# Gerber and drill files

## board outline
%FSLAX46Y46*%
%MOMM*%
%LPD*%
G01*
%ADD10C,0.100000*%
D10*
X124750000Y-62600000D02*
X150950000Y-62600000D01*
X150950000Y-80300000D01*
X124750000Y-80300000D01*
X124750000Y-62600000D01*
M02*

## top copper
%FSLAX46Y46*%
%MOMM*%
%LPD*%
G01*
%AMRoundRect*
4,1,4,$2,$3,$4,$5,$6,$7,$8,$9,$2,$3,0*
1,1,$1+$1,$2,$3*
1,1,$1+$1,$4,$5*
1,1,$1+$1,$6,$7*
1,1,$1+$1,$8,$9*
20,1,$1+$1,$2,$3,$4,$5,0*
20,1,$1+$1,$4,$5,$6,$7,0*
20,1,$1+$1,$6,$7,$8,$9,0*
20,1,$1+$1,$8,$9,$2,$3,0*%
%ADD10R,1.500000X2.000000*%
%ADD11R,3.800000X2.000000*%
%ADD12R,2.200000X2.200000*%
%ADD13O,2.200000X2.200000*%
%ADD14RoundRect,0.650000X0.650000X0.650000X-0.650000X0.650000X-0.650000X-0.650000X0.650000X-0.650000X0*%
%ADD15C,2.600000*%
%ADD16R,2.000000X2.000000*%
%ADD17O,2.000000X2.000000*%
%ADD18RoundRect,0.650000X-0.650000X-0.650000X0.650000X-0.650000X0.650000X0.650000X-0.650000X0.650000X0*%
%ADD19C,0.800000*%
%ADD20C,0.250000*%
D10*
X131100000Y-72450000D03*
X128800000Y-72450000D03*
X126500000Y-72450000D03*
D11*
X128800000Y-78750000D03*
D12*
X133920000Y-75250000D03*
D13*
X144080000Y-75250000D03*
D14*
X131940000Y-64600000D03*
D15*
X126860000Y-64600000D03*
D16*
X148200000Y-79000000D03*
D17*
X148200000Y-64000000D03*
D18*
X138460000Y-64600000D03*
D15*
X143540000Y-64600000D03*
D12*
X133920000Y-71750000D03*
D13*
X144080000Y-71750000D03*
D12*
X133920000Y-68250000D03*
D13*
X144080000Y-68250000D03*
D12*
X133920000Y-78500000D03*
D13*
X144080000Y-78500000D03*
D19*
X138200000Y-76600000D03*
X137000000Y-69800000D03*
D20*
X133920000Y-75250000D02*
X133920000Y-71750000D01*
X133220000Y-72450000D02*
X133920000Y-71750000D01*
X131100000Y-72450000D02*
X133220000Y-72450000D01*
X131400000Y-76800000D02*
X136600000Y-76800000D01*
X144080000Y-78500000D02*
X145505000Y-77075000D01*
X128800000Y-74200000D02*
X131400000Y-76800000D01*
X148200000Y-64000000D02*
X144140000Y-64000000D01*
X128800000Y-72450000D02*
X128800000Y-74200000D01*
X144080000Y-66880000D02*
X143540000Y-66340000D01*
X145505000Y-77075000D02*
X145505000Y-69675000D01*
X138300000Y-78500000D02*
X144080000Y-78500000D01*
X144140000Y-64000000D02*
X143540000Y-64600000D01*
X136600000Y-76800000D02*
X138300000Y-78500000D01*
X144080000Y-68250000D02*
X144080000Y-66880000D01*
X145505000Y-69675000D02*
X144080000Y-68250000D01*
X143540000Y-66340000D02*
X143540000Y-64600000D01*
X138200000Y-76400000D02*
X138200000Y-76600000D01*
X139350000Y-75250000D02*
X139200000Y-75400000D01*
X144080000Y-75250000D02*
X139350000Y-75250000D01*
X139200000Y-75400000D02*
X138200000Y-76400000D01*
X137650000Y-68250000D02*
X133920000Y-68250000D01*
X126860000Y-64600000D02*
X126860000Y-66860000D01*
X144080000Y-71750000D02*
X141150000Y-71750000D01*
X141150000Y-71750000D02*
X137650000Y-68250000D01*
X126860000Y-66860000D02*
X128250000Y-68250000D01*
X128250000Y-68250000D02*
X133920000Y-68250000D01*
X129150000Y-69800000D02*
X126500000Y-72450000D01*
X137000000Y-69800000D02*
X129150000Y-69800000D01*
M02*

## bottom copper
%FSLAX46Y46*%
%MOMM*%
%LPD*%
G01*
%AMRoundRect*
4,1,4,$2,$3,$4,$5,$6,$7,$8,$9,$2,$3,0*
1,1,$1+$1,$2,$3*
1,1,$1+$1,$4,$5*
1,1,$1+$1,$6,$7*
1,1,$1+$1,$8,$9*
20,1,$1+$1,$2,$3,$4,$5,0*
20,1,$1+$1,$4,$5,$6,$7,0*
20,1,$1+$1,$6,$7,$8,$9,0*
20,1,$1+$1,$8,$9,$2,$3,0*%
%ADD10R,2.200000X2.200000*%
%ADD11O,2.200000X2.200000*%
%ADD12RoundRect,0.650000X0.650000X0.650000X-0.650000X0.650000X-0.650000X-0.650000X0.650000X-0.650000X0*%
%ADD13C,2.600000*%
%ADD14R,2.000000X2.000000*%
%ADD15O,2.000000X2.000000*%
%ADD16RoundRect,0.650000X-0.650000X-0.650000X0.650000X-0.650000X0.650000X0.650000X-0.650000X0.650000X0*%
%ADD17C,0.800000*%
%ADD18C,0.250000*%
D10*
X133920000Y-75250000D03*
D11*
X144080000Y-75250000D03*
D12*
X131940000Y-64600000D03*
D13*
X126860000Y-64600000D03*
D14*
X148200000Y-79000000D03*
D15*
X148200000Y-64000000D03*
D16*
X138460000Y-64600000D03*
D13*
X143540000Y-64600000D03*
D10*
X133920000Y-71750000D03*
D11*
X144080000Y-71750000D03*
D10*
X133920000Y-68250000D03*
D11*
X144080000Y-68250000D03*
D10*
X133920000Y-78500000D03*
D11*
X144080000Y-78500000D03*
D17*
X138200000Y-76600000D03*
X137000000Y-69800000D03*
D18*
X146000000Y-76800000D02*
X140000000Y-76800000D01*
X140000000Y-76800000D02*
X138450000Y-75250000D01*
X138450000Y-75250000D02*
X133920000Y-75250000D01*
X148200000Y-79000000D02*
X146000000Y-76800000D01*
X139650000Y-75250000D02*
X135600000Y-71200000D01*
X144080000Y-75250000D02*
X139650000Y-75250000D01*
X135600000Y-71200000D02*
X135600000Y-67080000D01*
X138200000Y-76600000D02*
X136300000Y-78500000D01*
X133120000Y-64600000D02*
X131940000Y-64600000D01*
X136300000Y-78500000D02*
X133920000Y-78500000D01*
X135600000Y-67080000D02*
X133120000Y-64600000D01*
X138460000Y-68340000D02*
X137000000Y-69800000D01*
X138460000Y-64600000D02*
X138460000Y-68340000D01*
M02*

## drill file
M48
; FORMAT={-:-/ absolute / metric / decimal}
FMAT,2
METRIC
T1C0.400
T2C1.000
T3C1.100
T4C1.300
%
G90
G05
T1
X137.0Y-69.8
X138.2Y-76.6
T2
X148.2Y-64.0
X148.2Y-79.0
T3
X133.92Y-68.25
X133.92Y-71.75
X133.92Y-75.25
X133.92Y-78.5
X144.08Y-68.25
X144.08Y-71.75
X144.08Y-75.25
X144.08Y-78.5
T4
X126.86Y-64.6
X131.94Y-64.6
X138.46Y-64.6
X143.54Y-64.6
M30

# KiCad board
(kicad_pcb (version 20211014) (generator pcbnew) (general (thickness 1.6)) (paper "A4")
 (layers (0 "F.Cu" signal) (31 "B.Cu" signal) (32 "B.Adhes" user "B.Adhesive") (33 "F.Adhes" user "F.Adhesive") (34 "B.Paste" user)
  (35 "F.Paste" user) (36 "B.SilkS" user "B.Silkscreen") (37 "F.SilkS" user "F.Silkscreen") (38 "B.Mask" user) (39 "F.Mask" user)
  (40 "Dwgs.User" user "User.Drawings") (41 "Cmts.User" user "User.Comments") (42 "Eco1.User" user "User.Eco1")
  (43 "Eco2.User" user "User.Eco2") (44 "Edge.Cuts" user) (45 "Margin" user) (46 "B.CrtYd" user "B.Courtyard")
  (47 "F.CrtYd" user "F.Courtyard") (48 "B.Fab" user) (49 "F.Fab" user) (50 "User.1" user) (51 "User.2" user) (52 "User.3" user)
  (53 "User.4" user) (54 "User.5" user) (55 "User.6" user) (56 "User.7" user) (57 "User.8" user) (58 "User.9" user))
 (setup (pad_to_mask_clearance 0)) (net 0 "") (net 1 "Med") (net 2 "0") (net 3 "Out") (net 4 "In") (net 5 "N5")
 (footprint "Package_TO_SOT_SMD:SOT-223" (layer "F.Cu") (at 128.8 75.6 -90)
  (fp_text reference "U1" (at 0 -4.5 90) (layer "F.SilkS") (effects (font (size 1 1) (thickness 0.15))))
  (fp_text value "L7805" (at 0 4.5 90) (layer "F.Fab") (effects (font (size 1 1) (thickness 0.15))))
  (pad "1" smd rect (at -3.15 -2.3 270) (size 2 1.5) (layers "F.Cu" "F.Paste" "F.Mask") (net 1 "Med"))
  (pad "2" smd rect (at -3.15 0 270) (size 2 1.5) (layers "F.Cu" "F.Paste" "F.Mask") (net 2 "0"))
  (pad "3" smd rect (at -3.15 2.3 270) (size 2 1.5) (layers "F.Cu" "F.Paste" "F.Mask") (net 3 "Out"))
  (pad "4" smd rect (at 3.15 0 270) (size 2 3.8) (layers "F.Cu" "F.Paste" "F.Mask")))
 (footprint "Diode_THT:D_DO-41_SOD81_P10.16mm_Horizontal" (layer "F.Cu") (at 133.92 75.25)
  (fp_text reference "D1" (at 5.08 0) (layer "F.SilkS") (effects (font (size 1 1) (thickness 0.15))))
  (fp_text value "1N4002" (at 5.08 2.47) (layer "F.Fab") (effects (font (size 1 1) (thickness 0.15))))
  (pad "1" thru_hole rect (at 0 0) (size 2.2 2.2) (drill 1.1) (layers *.Cu *.Mask) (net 1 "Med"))
  (pad "2" thru_hole oval (at 10.16 0) (size 2.2 2.2) (drill 1.1) (layers *.Cu *.Mask) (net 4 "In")))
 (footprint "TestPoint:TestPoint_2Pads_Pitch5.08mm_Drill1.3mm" (layer "F.Cu") (at 131.94 64.6 180)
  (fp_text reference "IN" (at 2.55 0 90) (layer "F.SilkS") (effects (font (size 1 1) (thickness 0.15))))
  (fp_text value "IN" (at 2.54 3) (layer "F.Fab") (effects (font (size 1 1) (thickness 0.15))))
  (pad "1" thru_hole roundrect (at 0 0 180) (size 2.6 2.6) (drill 1.3) (layers *.Cu *.Mask) (roundrect_rratio 0.25) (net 4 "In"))
  (pad "2" thru_hole circle (at 5.08 0 180) (size 2.6 2.6) (drill 1.3) (layers *.Cu *.Mask) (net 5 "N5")))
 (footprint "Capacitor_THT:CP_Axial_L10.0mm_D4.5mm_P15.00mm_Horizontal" (layer "F.Cu") (at 148.2 79 90)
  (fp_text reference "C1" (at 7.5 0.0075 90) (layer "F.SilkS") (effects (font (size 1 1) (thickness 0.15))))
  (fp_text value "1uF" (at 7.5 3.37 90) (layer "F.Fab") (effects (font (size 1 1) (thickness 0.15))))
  (pad "1" thru_hole rect (at 0 0 90) (size 2 2) (drill 1) (layers *.Cu *.Mask) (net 1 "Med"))
  (pad "2" thru_hole oval (at 15 0 90) (size 2 2) (drill 1) (layers *.Cu *.Mask) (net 2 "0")))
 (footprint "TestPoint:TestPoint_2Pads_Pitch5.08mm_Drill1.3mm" (layer "F.Cu") (at 138.46 64.6)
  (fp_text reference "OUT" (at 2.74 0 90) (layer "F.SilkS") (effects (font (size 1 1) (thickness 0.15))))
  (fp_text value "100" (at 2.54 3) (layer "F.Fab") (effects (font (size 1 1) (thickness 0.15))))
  (pad "1" thru_hole roundrect (at 0 0) (size 2.6 2.6) (drill 1.3) (layers *.Cu *.Mask) (roundrect_rratio 0.25) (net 3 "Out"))
  (pad "2" thru_hole circle (at 5.08 0) (size 2.6 2.6) (drill 1.3) (layers *.Cu *.Mask) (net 2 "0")))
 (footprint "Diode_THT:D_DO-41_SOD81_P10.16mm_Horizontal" (layer "F.Cu") (at 133.92 71.75)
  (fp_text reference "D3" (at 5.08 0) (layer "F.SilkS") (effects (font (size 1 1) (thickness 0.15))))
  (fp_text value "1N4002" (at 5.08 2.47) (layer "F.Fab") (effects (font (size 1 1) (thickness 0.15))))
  (pad "1" thru_hole rect (at 0 0) (size 2.2 2.2) (drill 1.1) (layers *.Cu *.Mask) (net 1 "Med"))
  (pad "2" thru_hole oval (at 10.16 0) (size 2.2 2.2) (drill 1.1) (layers *.Cu *.Mask) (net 5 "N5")))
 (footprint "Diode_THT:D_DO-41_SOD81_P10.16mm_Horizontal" (layer "F.Cu") (at 133.92 68.25)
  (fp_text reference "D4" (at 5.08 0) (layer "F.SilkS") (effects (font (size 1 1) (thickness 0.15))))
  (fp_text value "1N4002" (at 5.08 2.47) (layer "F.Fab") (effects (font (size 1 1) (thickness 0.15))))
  (pad "1" thru_hole rect (at 0 0) (size 2.2 2.2) (drill 1.1) (layers *.Cu *.Mask) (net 5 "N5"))
  (pad "2" thru_hole oval (at 10.16 0) (size 2.2 2.2) (drill 1.1) (layers *.Cu *.Mask) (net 2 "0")))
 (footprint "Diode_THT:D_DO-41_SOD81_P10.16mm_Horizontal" (layer "F.Cu") (at 133.92 78.5)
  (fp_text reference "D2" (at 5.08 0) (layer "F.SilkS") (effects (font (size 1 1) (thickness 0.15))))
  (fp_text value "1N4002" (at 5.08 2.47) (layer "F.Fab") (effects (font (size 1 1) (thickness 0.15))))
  (pad "1" thru_hole rect (at 0 0) (size 2.2 2.2) (drill 1.1) (layers *.Cu *.Mask) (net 4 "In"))
  (pad "2" thru_hole oval (at 10.16 0) (size 2.2 2.2) (drill 1.1) (layers *.Cu *.Mask) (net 2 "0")))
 (gr_rect (start 150.95 62.6) (end 124.75 80.3) (layer "Edge.Cuts") (width 0.1) (fill none))
 (segment (start 133.92 75.25) (end 133.92 71.75) (width 0.25) (layer "F.Cu") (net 1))
 (segment (start 133.22 72.45) (end 133.92 71.75) (width 0.25) (layer "F.Cu") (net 1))
 (segment (start 131.1 72.45) (end 133.22 72.45) (width 0.25) (layer "F.Cu") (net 1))
 (segment (start 146 76.8) (end 140 76.8) (width 0.25) (layer "B.Cu") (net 1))
 (segment (start 140 76.8) (end 138.45 75.25) (width 0.25) (layer "B.Cu") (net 1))
 (segment (start 138.45 75.25) (end 133.92 75.25) (width 0.25) (layer "B.Cu") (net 1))
 (segment (start 148.2 79) (end 146 76.8) (width 0.25) (layer "B.Cu") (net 1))
 (segment (start 131.4 76.8) (end 136.6 76.8) (width 0.25) (layer "F.Cu") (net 2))
 (segment (start 144.08 78.5) (end 145.505 77.075) (width 0.25) (layer "F.Cu") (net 2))
 (segment (start 128.8 74.2) (end 131.4 76.8) (width 0.25) (layer "F.Cu") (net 2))
 (segment (start 148.2 64) (end 144.14 64) (width 0.25) (layer "F.Cu") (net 2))
 (segment (start 128.8 72.45) (end 128.8 74.2) (width 0.25) (layer "F.Cu") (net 2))
 (segment (start 144.08 66.88) (end 143.54 66.34) (width 0.25) (layer "F.Cu") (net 2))
 (segment (start 145.505 77.075) (end 145.505 69.675) (width 0.25) (layer "F.Cu") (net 2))
 (segment (start 138.3 78.5) (end 144.08 78.5) (width 0.25) (layer "F.Cu") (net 2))
 (segment (start 144.14 64) (end 143.54 64.6) (width 0.25) (layer "F.Cu") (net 2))
 (segment (start 136.6 76.8) (end 138.3 78.5) (width 0.25) (layer "F.Cu") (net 2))
 (segment (start 144.08 68.25) (end 144.08 66.88) (width 0.25) (layer "F.Cu") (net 2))
 (segment (start 145.505 69.675) (end 144.08 68.25) (width 0.25) (layer "F.Cu") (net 2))
 (segment (start 143.54 66.34) (end 143.54 64.6) (width 0.25) (layer "F.Cu") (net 2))
 (segment (start 138.2 76.4) (end 138.2 76.6) (width 0.25) (layer "F.Cu") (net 4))
 (segment (start 139.35 75.25) (end 139.2 75.4) (width 0.25) (layer "F.Cu") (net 4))
 (segment (start 144.08 75.25) (end 139.35 75.25) (width 0.25) (layer "F.Cu") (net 4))
 (segment (start 139.2 75.4) (end 138.2 76.4) (width 0.25) (layer "F.Cu") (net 4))
 (via (at 138.2 76.6) (size 0.8) (drill 0.4) (layers "F.Cu" "B.Cu") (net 4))
 (segment (start 139.65 75.25) (end 135.6 71.2) (width 0.25) (layer "B.Cu") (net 4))
 (segment (start 144.08 75.25) (end 139.65 75.25) (width 0.25) (layer "B.Cu") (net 4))
 (segment (start 135.6 71.2) (end 135.6 67.08) (width 0.25) (layer "B.Cu") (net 4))
 (segment (start 138.2 76.6) (end 136.3 78.5) (width 0.25) (layer "B.Cu") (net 4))
 (segment (start 133.12 64.6) (end 131.94 64.6) (width 0.25) (layer "B.Cu") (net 4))
 (segment (start 136.3 78.5) (end 133.92 78.5) (width 0.25) (layer "B.Cu") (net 4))
 (segment (start 135.6 67.08) (end 133.12 64.6) (width 0.25) (layer "B.Cu") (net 4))
 (segment (start 137.65 68.25) (end 133.92 68.25) (width 0.25) (layer "F.Cu") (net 5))
 (segment (start 126.86 64.6) (end 126.86 66.86) (width 0.25) (layer "F.Cu") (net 5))
 (segment (start 144.08 71.75) (end 141.15 71.75) (width 0.25) (layer "F.Cu") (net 5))
 (segment (start 141.15 71.75) (end 137.65 68.25) (width 0.25) (layer "F.Cu") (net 5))
 (segment (start 126.86 66.86) (end 128.25 68.25) (width 0.25) (layer "F.Cu") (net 5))
 (segment (start 128.25 68.25) (end 133.92 68.25) (width 0.25) (layer "F.Cu") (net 5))
 (segment (start 129.15 69.8) (end 126.5 72.45) (width 0.25) (layer "F.Cu") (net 3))
 (segment (start 137 69.8) (end 129.15 69.8) (width 0.25) (layer "F.Cu") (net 3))
 (via (at 137 69.8) (size 0.8) (drill 0.4) (layers "F.Cu" "B.Cu") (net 3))
 (segment (start 138.46 68.34) (end 137 69.8) (width 0.25) (layer "B.Cu") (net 3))
 (segment (start 138.46 64.6) (end 138.46 68.34) (width 0.25) (layer "B.Cu") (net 3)))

